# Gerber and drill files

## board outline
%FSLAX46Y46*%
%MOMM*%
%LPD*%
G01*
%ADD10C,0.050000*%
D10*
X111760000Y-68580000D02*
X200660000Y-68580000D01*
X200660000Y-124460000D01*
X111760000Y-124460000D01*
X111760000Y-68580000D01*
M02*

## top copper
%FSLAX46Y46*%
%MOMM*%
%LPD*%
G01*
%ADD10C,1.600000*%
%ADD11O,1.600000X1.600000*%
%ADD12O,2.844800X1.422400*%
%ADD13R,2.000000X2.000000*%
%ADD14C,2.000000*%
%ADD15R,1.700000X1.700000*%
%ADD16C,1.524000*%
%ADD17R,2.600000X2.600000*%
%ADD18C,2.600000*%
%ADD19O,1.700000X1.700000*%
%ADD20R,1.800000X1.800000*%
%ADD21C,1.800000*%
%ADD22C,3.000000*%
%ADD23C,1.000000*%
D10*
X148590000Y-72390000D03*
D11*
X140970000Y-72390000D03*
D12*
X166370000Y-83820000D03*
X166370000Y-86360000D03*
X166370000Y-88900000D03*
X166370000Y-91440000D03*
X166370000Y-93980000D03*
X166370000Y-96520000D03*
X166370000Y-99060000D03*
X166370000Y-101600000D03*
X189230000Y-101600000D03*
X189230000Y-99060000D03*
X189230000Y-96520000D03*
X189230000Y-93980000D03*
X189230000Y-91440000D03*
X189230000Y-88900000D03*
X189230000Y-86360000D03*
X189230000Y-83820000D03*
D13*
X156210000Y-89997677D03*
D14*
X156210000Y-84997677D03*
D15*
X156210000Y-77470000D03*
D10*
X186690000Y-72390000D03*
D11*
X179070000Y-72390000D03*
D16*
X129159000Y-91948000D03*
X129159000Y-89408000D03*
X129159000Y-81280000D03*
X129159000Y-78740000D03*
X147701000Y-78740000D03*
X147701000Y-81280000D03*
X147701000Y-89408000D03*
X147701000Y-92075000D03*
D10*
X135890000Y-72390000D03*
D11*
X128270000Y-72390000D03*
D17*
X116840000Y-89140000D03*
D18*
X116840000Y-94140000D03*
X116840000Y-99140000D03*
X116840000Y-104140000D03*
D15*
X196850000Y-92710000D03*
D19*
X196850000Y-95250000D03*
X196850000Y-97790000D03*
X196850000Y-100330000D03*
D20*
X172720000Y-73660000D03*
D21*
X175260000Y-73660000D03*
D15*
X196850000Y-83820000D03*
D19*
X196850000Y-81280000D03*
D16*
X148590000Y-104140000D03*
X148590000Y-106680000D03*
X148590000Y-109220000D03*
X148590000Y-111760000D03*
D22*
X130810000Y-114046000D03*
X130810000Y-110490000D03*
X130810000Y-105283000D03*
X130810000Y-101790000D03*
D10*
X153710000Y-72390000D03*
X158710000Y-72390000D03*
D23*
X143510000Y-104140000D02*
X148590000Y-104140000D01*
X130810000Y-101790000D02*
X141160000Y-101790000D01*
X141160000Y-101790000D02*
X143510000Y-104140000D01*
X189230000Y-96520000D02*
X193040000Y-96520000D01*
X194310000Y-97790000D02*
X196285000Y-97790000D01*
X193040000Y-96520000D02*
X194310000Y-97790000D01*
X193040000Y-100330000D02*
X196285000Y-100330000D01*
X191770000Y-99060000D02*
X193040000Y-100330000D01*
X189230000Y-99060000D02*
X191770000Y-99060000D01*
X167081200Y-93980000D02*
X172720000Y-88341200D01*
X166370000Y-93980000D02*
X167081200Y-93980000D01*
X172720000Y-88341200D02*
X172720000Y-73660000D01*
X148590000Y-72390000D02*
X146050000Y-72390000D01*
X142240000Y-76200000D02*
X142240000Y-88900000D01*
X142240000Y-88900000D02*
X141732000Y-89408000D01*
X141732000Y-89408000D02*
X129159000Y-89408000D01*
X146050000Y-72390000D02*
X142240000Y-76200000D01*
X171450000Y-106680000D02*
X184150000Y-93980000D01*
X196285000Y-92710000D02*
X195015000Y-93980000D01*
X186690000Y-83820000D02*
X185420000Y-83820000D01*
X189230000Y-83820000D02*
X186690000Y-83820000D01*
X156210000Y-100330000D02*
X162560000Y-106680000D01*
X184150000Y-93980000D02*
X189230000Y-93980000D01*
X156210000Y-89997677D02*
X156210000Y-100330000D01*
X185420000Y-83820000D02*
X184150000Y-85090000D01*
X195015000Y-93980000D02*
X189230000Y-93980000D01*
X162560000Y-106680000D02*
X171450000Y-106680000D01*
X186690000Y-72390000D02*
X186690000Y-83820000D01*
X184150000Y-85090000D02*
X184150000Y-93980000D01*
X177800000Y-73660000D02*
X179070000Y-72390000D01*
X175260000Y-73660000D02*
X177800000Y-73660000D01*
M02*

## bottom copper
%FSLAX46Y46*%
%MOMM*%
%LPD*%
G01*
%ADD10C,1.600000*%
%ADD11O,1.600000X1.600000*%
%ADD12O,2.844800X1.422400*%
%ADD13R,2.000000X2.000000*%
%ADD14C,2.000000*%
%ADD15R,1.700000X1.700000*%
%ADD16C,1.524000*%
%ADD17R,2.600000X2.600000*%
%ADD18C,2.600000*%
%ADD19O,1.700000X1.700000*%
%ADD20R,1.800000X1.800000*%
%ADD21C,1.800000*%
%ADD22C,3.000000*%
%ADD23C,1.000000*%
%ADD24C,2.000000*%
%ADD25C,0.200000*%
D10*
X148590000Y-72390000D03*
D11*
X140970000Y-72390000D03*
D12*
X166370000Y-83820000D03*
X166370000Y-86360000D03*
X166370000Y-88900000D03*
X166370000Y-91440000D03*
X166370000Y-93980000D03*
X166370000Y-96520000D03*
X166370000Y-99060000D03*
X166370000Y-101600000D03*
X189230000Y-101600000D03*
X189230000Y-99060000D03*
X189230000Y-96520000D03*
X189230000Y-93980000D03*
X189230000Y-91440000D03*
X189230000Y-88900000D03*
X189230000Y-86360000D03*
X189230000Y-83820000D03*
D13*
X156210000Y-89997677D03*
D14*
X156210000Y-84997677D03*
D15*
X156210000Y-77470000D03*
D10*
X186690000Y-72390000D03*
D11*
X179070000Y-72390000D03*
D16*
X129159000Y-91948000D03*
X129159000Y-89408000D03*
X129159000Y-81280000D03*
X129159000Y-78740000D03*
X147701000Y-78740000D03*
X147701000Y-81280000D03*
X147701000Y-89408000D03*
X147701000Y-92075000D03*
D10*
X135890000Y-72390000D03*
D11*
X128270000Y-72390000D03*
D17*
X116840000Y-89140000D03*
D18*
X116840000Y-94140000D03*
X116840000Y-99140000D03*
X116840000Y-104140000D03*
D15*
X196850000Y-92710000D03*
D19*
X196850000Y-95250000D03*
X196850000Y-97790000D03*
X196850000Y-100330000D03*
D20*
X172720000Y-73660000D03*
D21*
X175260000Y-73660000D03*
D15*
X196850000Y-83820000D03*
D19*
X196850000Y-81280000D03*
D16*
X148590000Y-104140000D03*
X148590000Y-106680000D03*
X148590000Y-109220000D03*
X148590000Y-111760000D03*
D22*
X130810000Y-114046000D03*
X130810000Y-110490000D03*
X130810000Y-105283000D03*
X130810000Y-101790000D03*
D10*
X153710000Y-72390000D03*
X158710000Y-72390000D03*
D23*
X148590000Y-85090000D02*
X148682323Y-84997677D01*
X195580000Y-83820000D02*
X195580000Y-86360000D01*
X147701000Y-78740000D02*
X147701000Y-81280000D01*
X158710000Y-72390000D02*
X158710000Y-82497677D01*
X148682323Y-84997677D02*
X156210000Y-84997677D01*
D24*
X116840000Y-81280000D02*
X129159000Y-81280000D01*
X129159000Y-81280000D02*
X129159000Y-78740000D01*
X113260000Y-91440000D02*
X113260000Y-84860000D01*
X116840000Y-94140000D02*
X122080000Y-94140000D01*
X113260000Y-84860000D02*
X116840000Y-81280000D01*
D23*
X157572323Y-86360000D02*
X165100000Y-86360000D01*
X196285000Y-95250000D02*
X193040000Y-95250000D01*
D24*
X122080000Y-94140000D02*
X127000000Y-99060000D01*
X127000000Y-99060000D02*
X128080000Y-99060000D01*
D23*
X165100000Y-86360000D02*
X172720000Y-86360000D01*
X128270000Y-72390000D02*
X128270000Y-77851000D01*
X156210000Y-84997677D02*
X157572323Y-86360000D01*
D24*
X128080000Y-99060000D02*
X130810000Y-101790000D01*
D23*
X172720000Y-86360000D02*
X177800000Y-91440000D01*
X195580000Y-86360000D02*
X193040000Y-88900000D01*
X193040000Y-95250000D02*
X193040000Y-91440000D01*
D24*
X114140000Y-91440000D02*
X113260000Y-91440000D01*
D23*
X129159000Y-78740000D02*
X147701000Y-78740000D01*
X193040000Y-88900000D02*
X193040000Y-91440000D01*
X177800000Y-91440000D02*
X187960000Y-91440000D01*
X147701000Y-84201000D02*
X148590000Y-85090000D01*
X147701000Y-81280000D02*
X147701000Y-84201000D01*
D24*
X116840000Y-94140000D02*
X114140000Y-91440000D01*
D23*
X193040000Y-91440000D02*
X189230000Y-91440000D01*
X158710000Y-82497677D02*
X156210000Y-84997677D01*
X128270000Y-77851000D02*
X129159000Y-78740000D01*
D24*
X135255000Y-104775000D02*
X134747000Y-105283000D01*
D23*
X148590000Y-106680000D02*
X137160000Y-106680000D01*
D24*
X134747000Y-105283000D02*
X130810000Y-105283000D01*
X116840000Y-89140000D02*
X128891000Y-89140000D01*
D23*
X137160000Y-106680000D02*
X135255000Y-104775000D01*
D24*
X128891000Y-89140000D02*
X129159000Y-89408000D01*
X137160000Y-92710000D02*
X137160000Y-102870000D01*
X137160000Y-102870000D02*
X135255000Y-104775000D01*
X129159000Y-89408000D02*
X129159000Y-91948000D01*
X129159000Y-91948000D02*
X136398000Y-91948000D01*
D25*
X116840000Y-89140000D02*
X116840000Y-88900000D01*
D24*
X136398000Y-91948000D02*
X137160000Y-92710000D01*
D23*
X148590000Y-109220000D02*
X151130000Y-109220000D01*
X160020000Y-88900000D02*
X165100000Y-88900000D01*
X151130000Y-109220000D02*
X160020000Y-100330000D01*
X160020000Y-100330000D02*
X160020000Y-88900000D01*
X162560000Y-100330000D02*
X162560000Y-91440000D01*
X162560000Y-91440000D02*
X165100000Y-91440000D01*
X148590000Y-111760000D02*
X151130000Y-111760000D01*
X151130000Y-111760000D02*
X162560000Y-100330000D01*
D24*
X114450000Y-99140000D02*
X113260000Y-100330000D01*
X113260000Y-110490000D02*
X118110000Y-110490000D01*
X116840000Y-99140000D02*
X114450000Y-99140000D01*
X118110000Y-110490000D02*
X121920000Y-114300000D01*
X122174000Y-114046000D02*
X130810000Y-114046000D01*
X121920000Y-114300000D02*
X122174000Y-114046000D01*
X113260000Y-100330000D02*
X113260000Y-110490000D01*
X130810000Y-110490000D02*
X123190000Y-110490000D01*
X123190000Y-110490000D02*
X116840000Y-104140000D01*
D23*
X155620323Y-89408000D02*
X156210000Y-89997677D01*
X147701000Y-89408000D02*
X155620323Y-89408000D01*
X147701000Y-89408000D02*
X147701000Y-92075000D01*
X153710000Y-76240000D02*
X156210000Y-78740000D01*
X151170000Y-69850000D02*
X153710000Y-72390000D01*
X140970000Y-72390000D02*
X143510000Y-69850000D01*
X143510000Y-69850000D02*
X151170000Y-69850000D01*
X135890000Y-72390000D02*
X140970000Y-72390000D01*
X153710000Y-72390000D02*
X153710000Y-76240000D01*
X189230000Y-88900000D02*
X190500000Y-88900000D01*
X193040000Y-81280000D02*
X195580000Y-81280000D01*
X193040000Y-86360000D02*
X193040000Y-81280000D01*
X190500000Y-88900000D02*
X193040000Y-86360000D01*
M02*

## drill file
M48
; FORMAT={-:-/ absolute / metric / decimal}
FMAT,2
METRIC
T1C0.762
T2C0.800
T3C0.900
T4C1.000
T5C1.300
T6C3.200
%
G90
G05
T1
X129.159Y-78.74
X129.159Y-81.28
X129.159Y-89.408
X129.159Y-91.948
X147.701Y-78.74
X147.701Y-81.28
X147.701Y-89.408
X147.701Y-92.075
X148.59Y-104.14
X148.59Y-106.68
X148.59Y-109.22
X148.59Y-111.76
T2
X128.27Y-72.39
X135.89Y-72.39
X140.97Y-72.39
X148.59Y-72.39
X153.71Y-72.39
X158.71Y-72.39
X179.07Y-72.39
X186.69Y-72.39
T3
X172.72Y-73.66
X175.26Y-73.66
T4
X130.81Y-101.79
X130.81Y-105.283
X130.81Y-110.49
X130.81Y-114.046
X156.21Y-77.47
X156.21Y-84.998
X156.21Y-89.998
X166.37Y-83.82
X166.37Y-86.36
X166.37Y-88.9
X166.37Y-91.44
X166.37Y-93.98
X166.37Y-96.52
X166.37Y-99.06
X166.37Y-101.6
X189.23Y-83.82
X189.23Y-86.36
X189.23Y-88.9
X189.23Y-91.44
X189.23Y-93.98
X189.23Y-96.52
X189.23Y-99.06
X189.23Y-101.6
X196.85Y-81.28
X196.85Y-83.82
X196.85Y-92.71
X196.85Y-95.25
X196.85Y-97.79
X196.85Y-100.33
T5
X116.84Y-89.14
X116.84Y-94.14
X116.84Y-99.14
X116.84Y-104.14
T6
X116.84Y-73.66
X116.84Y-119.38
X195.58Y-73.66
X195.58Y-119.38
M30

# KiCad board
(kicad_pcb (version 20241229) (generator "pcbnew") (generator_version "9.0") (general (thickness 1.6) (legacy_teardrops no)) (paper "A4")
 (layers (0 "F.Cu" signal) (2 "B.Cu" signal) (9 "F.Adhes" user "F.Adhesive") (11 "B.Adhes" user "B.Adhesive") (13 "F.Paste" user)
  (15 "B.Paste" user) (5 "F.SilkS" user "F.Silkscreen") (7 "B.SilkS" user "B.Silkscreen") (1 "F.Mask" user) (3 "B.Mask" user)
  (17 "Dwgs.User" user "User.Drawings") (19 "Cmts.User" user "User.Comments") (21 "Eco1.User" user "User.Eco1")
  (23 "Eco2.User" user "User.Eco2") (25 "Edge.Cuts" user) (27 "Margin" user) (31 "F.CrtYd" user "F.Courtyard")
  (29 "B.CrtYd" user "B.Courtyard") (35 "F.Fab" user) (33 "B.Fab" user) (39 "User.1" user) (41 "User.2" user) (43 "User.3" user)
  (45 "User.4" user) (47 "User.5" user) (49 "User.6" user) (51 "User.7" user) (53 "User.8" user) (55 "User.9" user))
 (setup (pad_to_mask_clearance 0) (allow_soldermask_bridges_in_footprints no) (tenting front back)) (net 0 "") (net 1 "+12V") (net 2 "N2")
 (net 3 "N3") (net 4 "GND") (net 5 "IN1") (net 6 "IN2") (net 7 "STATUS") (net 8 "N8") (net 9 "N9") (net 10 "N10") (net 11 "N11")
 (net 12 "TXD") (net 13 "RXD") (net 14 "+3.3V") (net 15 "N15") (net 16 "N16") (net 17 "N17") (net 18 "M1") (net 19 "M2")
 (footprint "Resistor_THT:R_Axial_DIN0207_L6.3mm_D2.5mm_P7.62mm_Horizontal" (layer "F.Cu") (at 148.59 72.39 180)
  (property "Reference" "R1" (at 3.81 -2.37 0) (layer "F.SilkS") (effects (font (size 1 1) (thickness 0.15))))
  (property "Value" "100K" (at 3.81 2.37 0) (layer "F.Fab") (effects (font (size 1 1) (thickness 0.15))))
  (pad "1" thru_hole circle (at 0 0 180) (size 1.6 1.6) (drill 0.8) (layers "*.Cu" "*.Mask") (remove_unused_layers no) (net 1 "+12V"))
  (pad "2" thru_hole oval (at 7.62 0 180) (size 1.6 1.6) (drill 0.8) (layers "*.Cu" "*.Mask") (remove_unused_layers no) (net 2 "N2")))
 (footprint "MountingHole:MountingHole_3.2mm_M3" (layer "F.Cu") (at 195.58 73.66)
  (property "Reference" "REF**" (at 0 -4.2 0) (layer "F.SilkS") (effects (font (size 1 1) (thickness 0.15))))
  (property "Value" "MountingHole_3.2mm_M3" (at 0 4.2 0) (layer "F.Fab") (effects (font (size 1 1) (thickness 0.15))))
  (pad "" np_thru_hole circle (at 0 0) (size 3.2 3.2) (drill 3.2) (layers "*.Cu" "*.Mask")))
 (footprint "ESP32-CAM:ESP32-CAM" (layer "F.Cu") (at 177.8 93.98)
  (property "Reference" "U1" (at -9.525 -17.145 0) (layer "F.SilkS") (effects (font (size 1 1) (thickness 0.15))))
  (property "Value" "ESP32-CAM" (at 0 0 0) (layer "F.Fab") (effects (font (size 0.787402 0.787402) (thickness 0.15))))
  (pad "P$1" thru_hole oval (at -11.43 -10.16) (size 2.8448 1.4224) (drill 1) (layers "*.Cu" "*.Mask") (remove_unused_layers no)
   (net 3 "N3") (solder_mask_margin 0.102))
  (pad "P$2" thru_hole oval (at -11.43 -7.62) (size 2.8448 1.4224) (drill 1) (layers "*.Cu" "*.Mask") (remove_unused_layers no)
   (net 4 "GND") (solder_mask_margin 0.102))
  (pad "P$3" thru_hole oval (at -11.43 -5.08) (size 2.8448 1.4224) (drill 1) (layers "*.Cu" "*.Mask") (remove_unused_layers no)
   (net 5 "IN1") (solder_mask_margin 0.102))
  (pad "P$4" thru_hole oval (at -11.43 -2.54) (size 2.8448 1.4224) (drill 1) (layers "*.Cu" "*.Mask") (remove_unused_layers no)
   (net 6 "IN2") (solder_mask_margin 0.102))
  (pad "P$5" thru_hole oval (at -11.43 0) (size 2.8448 1.4224) (drill 1) (layers "*.Cu" "*.Mask") (remove_unused_layers no) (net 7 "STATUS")
   (solder_mask_margin 0.102))
  (pad "P$6" thru_hole oval (at -11.43 2.54) (size 2.8448 1.4224) (drill 1) (layers "*.Cu" "*.Mask") (remove_unused_layers no) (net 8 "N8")
   (solder_mask_margin 0.102))
  (pad "P$7" thru_hole oval (at -11.43 5.08) (size 2.8448 1.4224) (drill 1) (layers "*.Cu" "*.Mask") (remove_unused_layers no) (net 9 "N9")
   (solder_mask_margin 0.102))
  (pad "P$8" thru_hole oval (at -11.43 7.62) (size 2.8448 1.4224) (drill 1) (layers "*.Cu" "*.Mask") (remove_unused_layers no)
   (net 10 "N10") (solder_mask_margin 0.102))
  (pad "P$9" thru_hole oval (at 11.43 7.62) (size 2.8448 1.4224) (drill 1) (layers "*.Cu" "*.Mask") (remove_unused_layers no) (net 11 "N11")
   (solder_mask_margin 0.102))
  (pad "P$10" thru_hole oval (at 11.43 5.08) (size 2.8448 1.4224) (drill 1) (layers "*.Cu" "*.Mask") (remove_unused_layers no)
   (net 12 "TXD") (solder_mask_margin 0.102))
  (pad "P$11" thru_hole oval (at 11.43 2.54) (size 2.8448 1.4224) (drill 1) (layers "*.Cu" "*.Mask") (remove_unused_layers no)
   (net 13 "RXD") (solder_mask_margin 0.102))
  (pad "P$12" thru_hole oval (at 11.43 0) (size 2.8448 1.4224) (drill 1) (layers "*.Cu" "*.Mask") (remove_unused_layers no) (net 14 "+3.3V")
   (solder_mask_margin 0.102))
  (pad "P$13" thru_hole oval (at 11.43 -2.54) (size 2.8448 1.4224) (drill 1) (layers "*.Cu" "*.Mask") (remove_unused_layers no)
   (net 4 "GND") (solder_mask_margin 0.102))
  (pad "P$14" thru_hole oval (at 11.43 -5.08) (size 2.8448 1.4224) (drill 1) (layers "*.Cu" "*.Mask") (remove_unused_layers no)
   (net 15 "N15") (solder_mask_margin 0.102))
  (pad "P$15" thru_hole oval (at 11.43 -7.62) (size 2.8448 1.4224) (drill 1) (layers "*.Cu" "*.Mask") (remove_unused_layers no)
   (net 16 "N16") (solder_mask_margin 0.102))
  (pad "P$16" thru_hole oval (at 11.43 -10.16) (size 2.8448 1.4224) (drill 1) (layers "*.Cu" "*.Mask") (remove_unused_layers no)
   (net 14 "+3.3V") (solder_mask_margin 0.102)))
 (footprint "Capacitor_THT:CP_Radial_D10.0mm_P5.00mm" (layer "F.Cu") (at 156.21 89.997677 90)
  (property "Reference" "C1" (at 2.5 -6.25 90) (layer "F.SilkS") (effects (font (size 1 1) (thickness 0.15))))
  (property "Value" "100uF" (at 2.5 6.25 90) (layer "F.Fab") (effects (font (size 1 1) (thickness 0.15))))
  (pad "1" thru_hole rect (at 0 0 90) (size 2 2) (drill 1) (layers "*.Cu" "*.Mask") (remove_unused_layers no) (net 14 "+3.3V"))
  (pad "2" thru_hole circle (at 5 0 90) (size 2 2) (drill 1) (layers "*.Cu" "*.Mask") (remove_unused_layers no) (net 4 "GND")))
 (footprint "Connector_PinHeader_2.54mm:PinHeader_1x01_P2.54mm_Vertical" (layer "F.Cu") (at 156.21 77.47)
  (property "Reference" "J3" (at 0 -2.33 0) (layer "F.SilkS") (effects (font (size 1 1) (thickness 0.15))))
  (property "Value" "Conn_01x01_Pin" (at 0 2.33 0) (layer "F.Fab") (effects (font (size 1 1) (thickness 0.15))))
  (pad "1" thru_hole rect (at 0 0) (size 1.7 1.7) (drill 1) (layers "*.Cu" "*.Mask") (remove_unused_layers no) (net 2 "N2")))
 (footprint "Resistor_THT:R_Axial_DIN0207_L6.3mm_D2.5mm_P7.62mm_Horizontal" (layer "F.Cu") (at 186.69 72.39 180)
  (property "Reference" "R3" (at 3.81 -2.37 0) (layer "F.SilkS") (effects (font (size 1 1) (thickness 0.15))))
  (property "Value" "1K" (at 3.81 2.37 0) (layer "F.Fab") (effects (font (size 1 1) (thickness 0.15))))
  (pad "1" thru_hole circle (at 0 0 180) (size 1.6 1.6) (drill 0.8) (layers "*.Cu" "*.Mask") (remove_unused_layers no) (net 14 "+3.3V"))
  (pad "2" thru_hole oval (at 7.62 0 180) (size 1.6 1.6) (drill 0.8) (layers "*.Cu" "*.Mask") (remove_unused_layers no) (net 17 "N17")))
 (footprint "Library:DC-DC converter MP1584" (layer "F.Cu") (at 129.159 91.948)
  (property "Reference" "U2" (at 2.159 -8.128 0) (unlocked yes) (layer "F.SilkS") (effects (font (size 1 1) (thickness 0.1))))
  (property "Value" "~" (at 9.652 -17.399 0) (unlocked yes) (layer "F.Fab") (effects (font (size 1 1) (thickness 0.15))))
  (pad "1" thru_hole circle (at 0 0) (size 1.524 1.524) (drill 0.762) (layers "*.Cu" "*.Mask") (remove_unused_layers no) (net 1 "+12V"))
  (pad "2" thru_hole circle (at 0 -2.54) (size 1.524 1.524) (drill 0.762) (layers "*.Cu" "*.Mask") (remove_unused_layers no) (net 1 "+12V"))
  (pad "3" thru_hole circle (at 0 -10.668) (size 1.524 1.524) (drill 0.762) (layers "*.Cu" "*.Mask") (remove_unused_layers no) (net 4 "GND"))
  (pad "4" thru_hole circle (at 0 -13.208) (size 1.524 1.524) (drill 0.762) (layers "*.Cu" "*.Mask") (remove_unused_layers no) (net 4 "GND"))
  (pad "5" thru_hole circle (at 18.542 -13.208) (size 1.524 1.524) (drill 0.762) (layers "*.Cu" "*.Mask") (remove_unused_layers no)
   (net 4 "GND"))
  (pad "6" thru_hole circle (at 18.542 -10.668) (size 1.524 1.524) (drill 0.762) (layers "*.Cu" "*.Mask") (remove_unused_layers no)
   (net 4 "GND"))
  (pad "7" thru_hole circle (at 18.542 -2.54) (size 1.524 1.524) (drill 0.762) (layers "*.Cu" "*.Mask") (remove_unused_layers no)
   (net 14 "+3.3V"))
  (pad "8" thru_hole circle (at 18.542 0.127) (size 1.524 1.524) (drill 0.762) (layers "*.Cu" "*.Mask") (remove_unused_layers no)
   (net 14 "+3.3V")))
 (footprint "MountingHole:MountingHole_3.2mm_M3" (layer "F.Cu") (at 116.84 119.38)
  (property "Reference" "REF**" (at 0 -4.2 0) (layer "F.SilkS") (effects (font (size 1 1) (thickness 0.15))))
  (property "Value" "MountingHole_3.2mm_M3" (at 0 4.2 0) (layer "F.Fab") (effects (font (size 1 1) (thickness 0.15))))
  (pad "" np_thru_hole circle (at 0 0) (size 3.2 3.2) (drill 3.2) (layers "*.Cu" "*.Mask")))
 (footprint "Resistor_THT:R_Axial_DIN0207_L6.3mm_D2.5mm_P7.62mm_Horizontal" (layer "F.Cu") (at 135.89 72.39 180)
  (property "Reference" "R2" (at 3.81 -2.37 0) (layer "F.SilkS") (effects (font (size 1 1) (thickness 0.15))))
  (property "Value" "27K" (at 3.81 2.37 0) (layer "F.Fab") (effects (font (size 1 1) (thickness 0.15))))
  (pad "1" thru_hole circle (at 0 0 180) (size 1.6 1.6) (drill 0.8) (layers "*.Cu" "*.Mask") (remove_unused_layers no) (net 2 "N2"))
  (pad "2" thru_hole oval (at 7.62 0 180) (size 1.6 1.6) (drill 0.8) (layers "*.Cu" "*.Mask") (remove_unused_layers no) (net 4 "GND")))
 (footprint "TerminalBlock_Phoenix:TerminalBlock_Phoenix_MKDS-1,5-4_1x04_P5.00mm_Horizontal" (layer "F.Cu") (at 116.84 89.14 -90)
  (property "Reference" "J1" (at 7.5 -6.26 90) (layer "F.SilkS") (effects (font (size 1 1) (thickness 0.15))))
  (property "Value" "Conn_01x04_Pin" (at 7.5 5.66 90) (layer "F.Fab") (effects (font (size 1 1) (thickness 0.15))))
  (pad "1" thru_hole rect (at 0 0 270) (size 2.6 2.6) (drill 1.3) (layers "*.Cu" "*.Mask") (remove_unused_layers no) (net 1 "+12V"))
  (pad "2" thru_hole circle (at 5 0 270) (size 2.6 2.6) (drill 1.3) (layers "*.Cu" "*.Mask") (remove_unused_layers no) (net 4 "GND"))
  (pad "3" thru_hole circle (at 10 0 270) (size 2.6 2.6) (drill 1.3) (layers "*.Cu" "*.Mask") (remove_unused_layers no) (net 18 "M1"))
  (pad "4" thru_hole circle (at 15 0 270) (size 2.6 2.6) (drill 1.3) (layers "*.Cu" "*.Mask") (remove_unused_layers no) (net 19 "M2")))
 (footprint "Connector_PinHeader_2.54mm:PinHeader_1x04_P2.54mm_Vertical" (layer "F.Cu") (at 196.85 92.71)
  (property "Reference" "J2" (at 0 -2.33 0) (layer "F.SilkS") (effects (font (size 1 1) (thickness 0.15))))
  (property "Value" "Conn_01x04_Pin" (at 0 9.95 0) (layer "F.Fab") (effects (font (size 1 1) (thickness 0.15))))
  (pad "1" thru_hole rect (at 0 0) (size 1.7 1.7) (drill 1) (layers "*.Cu" "*.Mask") (remove_unused_layers no) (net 14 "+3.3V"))
  (pad "2" thru_hole oval (at 0 2.54) (size 1.7 1.7) (drill 1) (layers "*.Cu" "*.Mask") (remove_unused_layers no) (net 4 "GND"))
  (pad "3" thru_hole oval (at 0 5.08) (size 1.7 1.7) (drill 1) (layers "*.Cu" "*.Mask") (remove_unused_layers no) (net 13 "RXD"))
  (pad "4" thru_hole oval (at 0 7.62) (size 1.7 1.7) (drill 1) (layers "*.Cu" "*.Mask") (remove_unused_layers no) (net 12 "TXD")))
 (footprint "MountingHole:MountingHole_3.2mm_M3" (layer "F.Cu") (at 116.84 73.66)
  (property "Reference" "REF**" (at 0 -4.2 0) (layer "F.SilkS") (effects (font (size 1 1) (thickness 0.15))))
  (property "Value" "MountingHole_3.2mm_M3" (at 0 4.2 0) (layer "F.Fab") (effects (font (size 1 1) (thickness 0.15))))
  (pad "" np_thru_hole circle (at 0 0) (size 3.2 3.2) (drill 3.2) (layers "*.Cu" "*.Mask")))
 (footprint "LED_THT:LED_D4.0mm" (layer "F.Cu") (at 172.72 73.66)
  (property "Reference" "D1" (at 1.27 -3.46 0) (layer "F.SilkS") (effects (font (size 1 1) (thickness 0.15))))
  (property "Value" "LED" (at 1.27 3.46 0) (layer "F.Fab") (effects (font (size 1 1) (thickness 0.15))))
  (pad "1" thru_hole rect (at 0 0) (size 1.8 1.8) (drill 0.9) (layers "*.Cu" "*.Mask") (remove_unused_layers no) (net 7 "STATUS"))
  (pad "2" thru_hole circle (at 2.54 0) (size 1.8 1.8) (drill 0.9) (layers "*.Cu" "*.Mask") (remove_unused_layers no) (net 17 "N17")))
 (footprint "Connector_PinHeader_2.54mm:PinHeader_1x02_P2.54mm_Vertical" (layer "F.Cu") (at 196.85 83.82 180)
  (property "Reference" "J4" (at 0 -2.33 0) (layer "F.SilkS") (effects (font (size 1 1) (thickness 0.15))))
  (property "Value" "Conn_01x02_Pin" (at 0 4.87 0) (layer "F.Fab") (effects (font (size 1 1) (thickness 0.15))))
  (pad "1" thru_hole rect (at 0 0 180) (size 1.7 1.7) (drill 1) (layers "*.Cu" "*.Mask") (remove_unused_layers no) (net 4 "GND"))
  (pad "2" thru_hole oval (at 0 2.54 180) (size 1.7 1.7) (drill 1) (layers "*.Cu" "*.Mask") (remove_unused_layers no) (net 15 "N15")))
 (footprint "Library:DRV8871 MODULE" (layer "F.Cu") (at 151.13 97.79 180)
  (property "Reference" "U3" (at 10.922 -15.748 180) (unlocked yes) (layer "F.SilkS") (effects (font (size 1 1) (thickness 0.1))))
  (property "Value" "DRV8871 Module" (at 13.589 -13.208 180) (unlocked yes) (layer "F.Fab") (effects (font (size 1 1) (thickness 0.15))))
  (pad "1" thru_hole circle (at 2.54 -6.35 180) (size 1.524 1.524) (drill 0.762) (layers "*.Cu" "*.Mask") (remove_unused_layers no)
   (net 4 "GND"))
  (pad "2" thru_hole circle (at 2.54 -8.89 180) (size 1.524 1.524) (drill 0.762) (layers "*.Cu" "*.Mask") (remove_unused_layers no)
   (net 1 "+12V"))
  (pad "3" thru_hole circle (at 2.54 -11.43 180) (size 1.524 1.524) (drill 0.762) (layers "*.Cu" "*.Mask") (remove_unused_layers no)
   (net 5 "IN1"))
  (pad "4" thru_hole circle (at 2.54 -13.97 180) (size 1.524 1.524) (drill 0.762) (layers "*.Cu" "*.Mask") (remove_unused_layers no)
   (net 6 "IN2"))
  (pad "5" thru_hole circle (at 20.32 -16.256 180) (size 3 3) (drill 1) (layers "*.Cu" "*.Mask") (remove_unused_layers no) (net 18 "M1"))
  (pad "6" thru_hole circle (at 20.32 -12.7 180) (size 3 3) (drill 1) (layers "*.Cu" "*.Mask") (remove_unused_layers no) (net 19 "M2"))
  (pad "7" thru_hole circle (at 20.32 -7.493 180) (size 3 3) (drill 1) (layers "*.Cu" "*.Mask") (remove_unused_layers no) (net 1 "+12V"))
  (pad "8" thru_hole circle (at 20.32 -4 180) (size 3 3) (drill 1) (layers "*.Cu" "*.Mask") (remove_unused_layers no) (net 4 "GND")))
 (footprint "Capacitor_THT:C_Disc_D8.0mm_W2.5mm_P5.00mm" (layer "F.Cu") (at 153.71 72.39)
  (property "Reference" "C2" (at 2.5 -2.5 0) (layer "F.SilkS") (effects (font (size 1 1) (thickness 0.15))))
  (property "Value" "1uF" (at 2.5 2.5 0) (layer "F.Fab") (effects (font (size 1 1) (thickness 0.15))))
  (pad "1" thru_hole circle (at 0 0) (size 1.6 1.6) (drill 0.8) (layers "*.Cu" "*.Mask") (remove_unused_layers no) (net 2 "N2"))
  (pad "2" thru_hole circle (at 5 0) (size 1.6 1.6) (drill 0.8) (layers "*.Cu" "*.Mask") (remove_unused_layers no) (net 4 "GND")))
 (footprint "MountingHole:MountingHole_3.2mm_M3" (layer "F.Cu") (at 195.58 119.38)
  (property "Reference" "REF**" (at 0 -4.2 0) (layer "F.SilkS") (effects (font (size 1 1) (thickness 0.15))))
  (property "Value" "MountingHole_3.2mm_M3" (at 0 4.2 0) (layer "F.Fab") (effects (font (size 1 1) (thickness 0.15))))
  (pad "" np_thru_hole circle (at 0 0) (size 3.2 3.2) (drill 3.2) (layers "*.Cu" "*.Mask")))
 (gr_rect (start 111.76 68.58) (end 200.66 124.46) (stroke (width 0.05) (type default)) (fill no) (layer "Edge.Cuts"))
 (segment (start 143.51 104.14) (end 148.59 104.14) (width 1) (layer "F.Cu") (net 4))
 (segment (start 130.81 101.79) (end 141.16 101.79) (width 1) (layer "F.Cu") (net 4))
 (segment (start 141.16 101.79) (end 143.51 104.14) (width 1) (layer "F.Cu") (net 4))
 (segment (start 148.59 85.09) (end 148.682323 84.997677) (width 1) (layer "B.Cu") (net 4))
 (segment (start 195.58 83.82) (end 195.58 86.36) (width 1) (layer "B.Cu") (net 4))
 (segment (start 147.701 78.74) (end 147.701 81.28) (width 1) (layer "B.Cu") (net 4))
 (segment (start 158.71 72.39) (end 158.71 82.497677) (width 1) (layer "B.Cu") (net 4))
 (segment (start 148.682323 84.997677) (end 156.21 84.997677) (width 1) (layer "B.Cu") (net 4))
 (segment (start 116.84 81.28) (end 129.159 81.28) (width 2) (layer "B.Cu") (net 4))
 (segment (start 129.159 81.28) (end 129.159 78.74) (width 2) (layer "B.Cu") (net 4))
 (segment (start 113.26 91.44) (end 113.26 84.86) (width 2) (layer "B.Cu") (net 4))
 (segment (start 116.84 94.14) (end 122.08 94.14) (width 2) (layer "B.Cu") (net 4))
 (segment (start 113.26 84.86) (end 116.84 81.28) (width 2) (layer "B.Cu") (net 4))
 (segment (start 157.572323 86.36) (end 165.1 86.36) (width 1) (layer "B.Cu") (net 4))
 (segment (start 196.285 95.25) (end 193.04 95.25) (width 1) (layer "B.Cu") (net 4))
 (segment (start 122.08 94.14) (end 127 99.06) (width 2) (layer "B.Cu") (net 4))
 (segment (start 127 99.06) (end 128.08 99.06) (width 2) (layer "B.Cu") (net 4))
 (segment (start 165.1 86.36) (end 172.72 86.36) (width 1) (layer "B.Cu") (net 4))
 (segment (start 128.27 72.39) (end 128.27 77.851) (width 1) (layer "B.Cu") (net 4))
 (segment (start 156.21 84.997677) (end 157.572323 86.36) (width 1) (layer "B.Cu") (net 4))
 (segment (start 128.08 99.06) (end 130.81 101.79) (width 2) (layer "B.Cu") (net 4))
 (segment (start 172.72 86.36) (end 177.8 91.44) (width 1) (layer "B.Cu") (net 4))
 (segment (start 195.58 86.36) (end 193.04 88.9) (width 1) (layer "B.Cu") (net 4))
 (segment (start 193.04 95.25) (end 193.04 91.44) (width 1) (layer "B.Cu") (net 4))
 (segment (start 114.14 91.44) (end 113.26 91.44) (width 2) (layer "B.Cu") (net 4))
 (segment (start 129.159 78.74) (end 147.701 78.74) (width 1) (layer "B.Cu") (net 4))
 (segment (start 193.04 88.9) (end 193.04 91.44) (width 1) (layer "B.Cu") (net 4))
 (segment (start 177.8 91.44) (end 187.96 91.44) (width 1) (layer "B.Cu") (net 4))
 (segment (start 147.701 84.201) (end 148.59 85.09) (width 1) (layer "B.Cu") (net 4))
 (segment (start 147.701 81.28) (end 147.701 84.201) (width 1) (layer "B.Cu") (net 4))
 (segment (start 116.84 94.14) (end 114.14 91.44) (width 2) (layer "B.Cu") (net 4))
 (segment (start 193.04 91.44) (end 189.23 91.44) (width 1) (layer "B.Cu") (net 4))
 (segment (start 158.71 82.497677) (end 156.21 84.997677) (width 1) (layer "B.Cu") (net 4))
 (segment (start 128.27 77.851) (end 129.159 78.74) (width 1) (layer "B.Cu") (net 4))
 (segment (start 189.23 96.52) (end 193.04 96.52) (width 1) (layer "F.Cu") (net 13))
 (segment (start 194.31 97.79) (end 196.285 97.79) (width 1) (layer "F.Cu") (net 13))
 (segment (start 193.04 96.52) (end 194.31 97.79) (width 1) (layer "F.Cu") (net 13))
 (segment (start 193.04 100.33) (end 196.285 100.33) (width 1) (layer "F.Cu") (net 12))
 (segment (start 191.77 99.06) (end 193.04 100.33) (width 1) (layer "F.Cu") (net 12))
 (segment (start 189.23 99.06) (end 191.77 99.06) (width 1) (layer "F.Cu") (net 12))
 (segment (start 167.0812 93.98) (end 172.72 88.3412) (width 1) (layer "F.Cu") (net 7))
 (segment (start 166.37 93.98) (end 167.0812 93.98) (width 1) (layer "F.Cu") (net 7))
 (segment (start 172.72 88.3412) (end 172.72 73.66) (width 1) (layer "F.Cu") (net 7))
 (segment (start 148.59 72.39) (end 146.05 72.39) (width 1) (layer "F.Cu") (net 1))
 (segment (start 142.24 76.2) (end 142.24 88.9) (width 1) (layer "F.Cu") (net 1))
 (segment (start 142.24 88.9) (end 141.732 89.408) (width 1) (layer "F.Cu") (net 1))
 (segment (start 141.732 89.408) (end 129.159 89.408) (width 1) (layer "F.Cu") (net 1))
 (segment (start 146.05 72.39) (end 142.24 76.2) (width 1) (layer "F.Cu") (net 1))
 (segment (start 135.255 104.775) (end 134.747 105.283) (width 2) (layer "B.Cu") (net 1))
 (segment (start 148.59 106.68) (end 137.16 106.68) (width 1) (layer "B.Cu") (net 1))
 (segment (start 134.747 105.283) (end 130.81 105.283) (width 2) (layer "B.Cu") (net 1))
 (segment (start 116.84 89.14) (end 128.891 89.14) (width 2) (layer "B.Cu") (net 1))
 (segment (start 137.16 106.68) (end 135.255 104.775) (width 1) (layer "B.Cu") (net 1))
 (segment (start 128.891 89.14) (end 129.159 89.408) (width 2) (layer "B.Cu") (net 1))
 (segment (start 137.16 92.71) (end 137.16 102.87) (width 2) (layer "B.Cu") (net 1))
 (segment (start 137.16 102.87) (end 135.255 104.775) (width 2) (layer "B.Cu") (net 1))
 (segment (start 129.159 89.408) (end 129.159 91.948) (width 2) (layer "B.Cu") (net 1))
 (segment (start 129.159 91.948) (end 136.398 91.948) (width 2) (layer "B.Cu") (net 1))
 (segment (start 116.84 89.14) (end 116.84 88.9) (width 0.2) (layer "B.Cu") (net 1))
 (segment (start 136.398 91.948) (end 137.16 92.71) (width 2) (layer "B.Cu") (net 1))
 (segment (start 148.59 109.22) (end 151.13 109.22) (width 1) (layer "B.Cu") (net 5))
 (segment (start 160.02 88.9) (end 165.1 88.9) (width 1) (layer "B.Cu") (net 5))
 (segment (start 151.13 109.22) (end 160.02 100.33) (width 1) (layer "B.Cu") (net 5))
 (segment (start 160.02 100.33) (end 160.02 88.9) (width 1) (layer "B.Cu") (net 5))
 (segment (start 162.56 100.33) (end 162.56 91.44) (width 1) (layer "B.Cu") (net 6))
 (segment (start 162.56 91.44) (end 165.1 91.44) (width 1) (layer "B.Cu") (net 6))
 (segment (start 148.59 111.76) (end 151.13 111.76) (width 1) (layer "B.Cu") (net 6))
 (segment (start 151.13 111.76) (end 162.56 100.33) (width 1) (layer "B.Cu") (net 6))
 (segment (start 114.45 99.14) (end 113.26 100.33) (width 2) (layer "B.Cu") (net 18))
 (segment (start 113.26 110.49) (end 118.11 110.49) (width 2) (layer "B.Cu") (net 18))
 (segment (start 116.84 99.14) (end 114.45 99.14) (width 2) (layer "B.Cu") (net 18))
 (segment (start 118.11 110.49) (end 121.92 114.3) (width 2) (layer "B.Cu") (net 18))
 (segment (start 122.174 114.046) (end 130.81 114.046) (width 2) (layer "B.Cu") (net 18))
 (segment (start 121.92 114.3) (end 122.174 114.046) (width 2) (layer "B.Cu") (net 18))
 (segment (start 113.26 100.33) (end 113.26 110.49) (width 2) (layer "B.Cu") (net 18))
 (segment (start 130.81 110.49) (end 123.19 110.49) (width 2) (layer "B.Cu") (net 19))
 (segment (start 123.19 110.49) (end 116.84 104.14) (width 2) (layer "B.Cu") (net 19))
 (segment (start 171.45 106.68) (end 184.15 93.98) (width 1) (layer "F.Cu") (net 14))
 (segment (start 196.285 92.71) (end 195.015 93.98) (width 1) (layer "F.Cu") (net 14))
 (segment (start 186.69 83.82) (end 185.42 83.82) (width 1) (layer "F.Cu") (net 14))
 (segment (start 189.23 83.82) (end 186.69 83.82) (width 1) (layer "F.Cu") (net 14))
 (segment (start 156.21 100.33) (end 162.56 106.68) (width 1) (layer "F.Cu") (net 14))
 (segment (start 184.15 93.98) (end 189.23 93.98) (width 1) (layer "F.Cu") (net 14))
 (segment (start 156.21 89.997677) (end 156.21 100.33) (width 1) (layer "F.Cu") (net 14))
 (segment (start 185.42 83.82) (end 184.15 85.09) (width 1) (layer "F.Cu") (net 14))
 (segment (start 195.015 93.98) (end 189.23 93.98) (width 1) (layer "F.Cu") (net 14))
 (segment (start 162.56 106.68) (end 171.45 106.68) (width 1) (layer "F.Cu") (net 14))
 (segment (start 186.69 72.39) (end 186.69 83.82) (width 1) (layer "F.Cu") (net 14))
 (segment (start 184.15 85.09) (end 184.15 93.98) (width 1) (layer "F.Cu") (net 14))
 (segment (start 155.620323 89.408) (end 156.21 89.997677) (width 1) (layer "B.Cu") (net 14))
 (segment (start 147.701 89.408) (end 155.620323 89.408) (width 1) (layer "B.Cu") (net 14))
 (segment (start 147.701 89.408) (end 147.701 92.075) (width 1) (layer "B.Cu") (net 14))
 (segment (start 153.71 76.24) (end 156.21 78.74) (width 1) (layer "B.Cu") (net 2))
 (segment (start 151.17 69.85) (end 153.71 72.39) (width 1) (layer "B.Cu") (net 2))
 (segment (start 140.97 72.39) (end 143.51 69.85) (width 1) (layer "B.Cu") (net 2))
 (segment (start 143.51 69.85) (end 151.17 69.85) (width 1) (layer "B.Cu") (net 2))
 (segment (start 135.89 72.39) (end 140.97 72.39) (width 1) (layer "B.Cu") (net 2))
 (segment (start 153.71 72.39) (end 153.71 76.24) (width 1) (layer "B.Cu") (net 2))
 (segment (start 189.23 88.9) (end 190.5 88.9) (width 1) (layer "B.Cu") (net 15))
 (segment (start 193.04 81.28) (end 195.58 81.28) (width 1) (layer "B.Cu") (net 15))
 (segment (start 193.04 86.36) (end 193.04 81.28) (width 1) (layer "B.Cu") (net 15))
 (segment (start 190.5 88.9) (end 193.04 86.36) (width 1) (layer "B.Cu") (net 15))
 (segment (start 177.8 73.66) (end 179.07 72.39) (width 1) (layer "F.Cu") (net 17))
 (segment (start 175.26 73.66) (end 177.8 73.66) (width 1) (layer "F.Cu") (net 17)))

